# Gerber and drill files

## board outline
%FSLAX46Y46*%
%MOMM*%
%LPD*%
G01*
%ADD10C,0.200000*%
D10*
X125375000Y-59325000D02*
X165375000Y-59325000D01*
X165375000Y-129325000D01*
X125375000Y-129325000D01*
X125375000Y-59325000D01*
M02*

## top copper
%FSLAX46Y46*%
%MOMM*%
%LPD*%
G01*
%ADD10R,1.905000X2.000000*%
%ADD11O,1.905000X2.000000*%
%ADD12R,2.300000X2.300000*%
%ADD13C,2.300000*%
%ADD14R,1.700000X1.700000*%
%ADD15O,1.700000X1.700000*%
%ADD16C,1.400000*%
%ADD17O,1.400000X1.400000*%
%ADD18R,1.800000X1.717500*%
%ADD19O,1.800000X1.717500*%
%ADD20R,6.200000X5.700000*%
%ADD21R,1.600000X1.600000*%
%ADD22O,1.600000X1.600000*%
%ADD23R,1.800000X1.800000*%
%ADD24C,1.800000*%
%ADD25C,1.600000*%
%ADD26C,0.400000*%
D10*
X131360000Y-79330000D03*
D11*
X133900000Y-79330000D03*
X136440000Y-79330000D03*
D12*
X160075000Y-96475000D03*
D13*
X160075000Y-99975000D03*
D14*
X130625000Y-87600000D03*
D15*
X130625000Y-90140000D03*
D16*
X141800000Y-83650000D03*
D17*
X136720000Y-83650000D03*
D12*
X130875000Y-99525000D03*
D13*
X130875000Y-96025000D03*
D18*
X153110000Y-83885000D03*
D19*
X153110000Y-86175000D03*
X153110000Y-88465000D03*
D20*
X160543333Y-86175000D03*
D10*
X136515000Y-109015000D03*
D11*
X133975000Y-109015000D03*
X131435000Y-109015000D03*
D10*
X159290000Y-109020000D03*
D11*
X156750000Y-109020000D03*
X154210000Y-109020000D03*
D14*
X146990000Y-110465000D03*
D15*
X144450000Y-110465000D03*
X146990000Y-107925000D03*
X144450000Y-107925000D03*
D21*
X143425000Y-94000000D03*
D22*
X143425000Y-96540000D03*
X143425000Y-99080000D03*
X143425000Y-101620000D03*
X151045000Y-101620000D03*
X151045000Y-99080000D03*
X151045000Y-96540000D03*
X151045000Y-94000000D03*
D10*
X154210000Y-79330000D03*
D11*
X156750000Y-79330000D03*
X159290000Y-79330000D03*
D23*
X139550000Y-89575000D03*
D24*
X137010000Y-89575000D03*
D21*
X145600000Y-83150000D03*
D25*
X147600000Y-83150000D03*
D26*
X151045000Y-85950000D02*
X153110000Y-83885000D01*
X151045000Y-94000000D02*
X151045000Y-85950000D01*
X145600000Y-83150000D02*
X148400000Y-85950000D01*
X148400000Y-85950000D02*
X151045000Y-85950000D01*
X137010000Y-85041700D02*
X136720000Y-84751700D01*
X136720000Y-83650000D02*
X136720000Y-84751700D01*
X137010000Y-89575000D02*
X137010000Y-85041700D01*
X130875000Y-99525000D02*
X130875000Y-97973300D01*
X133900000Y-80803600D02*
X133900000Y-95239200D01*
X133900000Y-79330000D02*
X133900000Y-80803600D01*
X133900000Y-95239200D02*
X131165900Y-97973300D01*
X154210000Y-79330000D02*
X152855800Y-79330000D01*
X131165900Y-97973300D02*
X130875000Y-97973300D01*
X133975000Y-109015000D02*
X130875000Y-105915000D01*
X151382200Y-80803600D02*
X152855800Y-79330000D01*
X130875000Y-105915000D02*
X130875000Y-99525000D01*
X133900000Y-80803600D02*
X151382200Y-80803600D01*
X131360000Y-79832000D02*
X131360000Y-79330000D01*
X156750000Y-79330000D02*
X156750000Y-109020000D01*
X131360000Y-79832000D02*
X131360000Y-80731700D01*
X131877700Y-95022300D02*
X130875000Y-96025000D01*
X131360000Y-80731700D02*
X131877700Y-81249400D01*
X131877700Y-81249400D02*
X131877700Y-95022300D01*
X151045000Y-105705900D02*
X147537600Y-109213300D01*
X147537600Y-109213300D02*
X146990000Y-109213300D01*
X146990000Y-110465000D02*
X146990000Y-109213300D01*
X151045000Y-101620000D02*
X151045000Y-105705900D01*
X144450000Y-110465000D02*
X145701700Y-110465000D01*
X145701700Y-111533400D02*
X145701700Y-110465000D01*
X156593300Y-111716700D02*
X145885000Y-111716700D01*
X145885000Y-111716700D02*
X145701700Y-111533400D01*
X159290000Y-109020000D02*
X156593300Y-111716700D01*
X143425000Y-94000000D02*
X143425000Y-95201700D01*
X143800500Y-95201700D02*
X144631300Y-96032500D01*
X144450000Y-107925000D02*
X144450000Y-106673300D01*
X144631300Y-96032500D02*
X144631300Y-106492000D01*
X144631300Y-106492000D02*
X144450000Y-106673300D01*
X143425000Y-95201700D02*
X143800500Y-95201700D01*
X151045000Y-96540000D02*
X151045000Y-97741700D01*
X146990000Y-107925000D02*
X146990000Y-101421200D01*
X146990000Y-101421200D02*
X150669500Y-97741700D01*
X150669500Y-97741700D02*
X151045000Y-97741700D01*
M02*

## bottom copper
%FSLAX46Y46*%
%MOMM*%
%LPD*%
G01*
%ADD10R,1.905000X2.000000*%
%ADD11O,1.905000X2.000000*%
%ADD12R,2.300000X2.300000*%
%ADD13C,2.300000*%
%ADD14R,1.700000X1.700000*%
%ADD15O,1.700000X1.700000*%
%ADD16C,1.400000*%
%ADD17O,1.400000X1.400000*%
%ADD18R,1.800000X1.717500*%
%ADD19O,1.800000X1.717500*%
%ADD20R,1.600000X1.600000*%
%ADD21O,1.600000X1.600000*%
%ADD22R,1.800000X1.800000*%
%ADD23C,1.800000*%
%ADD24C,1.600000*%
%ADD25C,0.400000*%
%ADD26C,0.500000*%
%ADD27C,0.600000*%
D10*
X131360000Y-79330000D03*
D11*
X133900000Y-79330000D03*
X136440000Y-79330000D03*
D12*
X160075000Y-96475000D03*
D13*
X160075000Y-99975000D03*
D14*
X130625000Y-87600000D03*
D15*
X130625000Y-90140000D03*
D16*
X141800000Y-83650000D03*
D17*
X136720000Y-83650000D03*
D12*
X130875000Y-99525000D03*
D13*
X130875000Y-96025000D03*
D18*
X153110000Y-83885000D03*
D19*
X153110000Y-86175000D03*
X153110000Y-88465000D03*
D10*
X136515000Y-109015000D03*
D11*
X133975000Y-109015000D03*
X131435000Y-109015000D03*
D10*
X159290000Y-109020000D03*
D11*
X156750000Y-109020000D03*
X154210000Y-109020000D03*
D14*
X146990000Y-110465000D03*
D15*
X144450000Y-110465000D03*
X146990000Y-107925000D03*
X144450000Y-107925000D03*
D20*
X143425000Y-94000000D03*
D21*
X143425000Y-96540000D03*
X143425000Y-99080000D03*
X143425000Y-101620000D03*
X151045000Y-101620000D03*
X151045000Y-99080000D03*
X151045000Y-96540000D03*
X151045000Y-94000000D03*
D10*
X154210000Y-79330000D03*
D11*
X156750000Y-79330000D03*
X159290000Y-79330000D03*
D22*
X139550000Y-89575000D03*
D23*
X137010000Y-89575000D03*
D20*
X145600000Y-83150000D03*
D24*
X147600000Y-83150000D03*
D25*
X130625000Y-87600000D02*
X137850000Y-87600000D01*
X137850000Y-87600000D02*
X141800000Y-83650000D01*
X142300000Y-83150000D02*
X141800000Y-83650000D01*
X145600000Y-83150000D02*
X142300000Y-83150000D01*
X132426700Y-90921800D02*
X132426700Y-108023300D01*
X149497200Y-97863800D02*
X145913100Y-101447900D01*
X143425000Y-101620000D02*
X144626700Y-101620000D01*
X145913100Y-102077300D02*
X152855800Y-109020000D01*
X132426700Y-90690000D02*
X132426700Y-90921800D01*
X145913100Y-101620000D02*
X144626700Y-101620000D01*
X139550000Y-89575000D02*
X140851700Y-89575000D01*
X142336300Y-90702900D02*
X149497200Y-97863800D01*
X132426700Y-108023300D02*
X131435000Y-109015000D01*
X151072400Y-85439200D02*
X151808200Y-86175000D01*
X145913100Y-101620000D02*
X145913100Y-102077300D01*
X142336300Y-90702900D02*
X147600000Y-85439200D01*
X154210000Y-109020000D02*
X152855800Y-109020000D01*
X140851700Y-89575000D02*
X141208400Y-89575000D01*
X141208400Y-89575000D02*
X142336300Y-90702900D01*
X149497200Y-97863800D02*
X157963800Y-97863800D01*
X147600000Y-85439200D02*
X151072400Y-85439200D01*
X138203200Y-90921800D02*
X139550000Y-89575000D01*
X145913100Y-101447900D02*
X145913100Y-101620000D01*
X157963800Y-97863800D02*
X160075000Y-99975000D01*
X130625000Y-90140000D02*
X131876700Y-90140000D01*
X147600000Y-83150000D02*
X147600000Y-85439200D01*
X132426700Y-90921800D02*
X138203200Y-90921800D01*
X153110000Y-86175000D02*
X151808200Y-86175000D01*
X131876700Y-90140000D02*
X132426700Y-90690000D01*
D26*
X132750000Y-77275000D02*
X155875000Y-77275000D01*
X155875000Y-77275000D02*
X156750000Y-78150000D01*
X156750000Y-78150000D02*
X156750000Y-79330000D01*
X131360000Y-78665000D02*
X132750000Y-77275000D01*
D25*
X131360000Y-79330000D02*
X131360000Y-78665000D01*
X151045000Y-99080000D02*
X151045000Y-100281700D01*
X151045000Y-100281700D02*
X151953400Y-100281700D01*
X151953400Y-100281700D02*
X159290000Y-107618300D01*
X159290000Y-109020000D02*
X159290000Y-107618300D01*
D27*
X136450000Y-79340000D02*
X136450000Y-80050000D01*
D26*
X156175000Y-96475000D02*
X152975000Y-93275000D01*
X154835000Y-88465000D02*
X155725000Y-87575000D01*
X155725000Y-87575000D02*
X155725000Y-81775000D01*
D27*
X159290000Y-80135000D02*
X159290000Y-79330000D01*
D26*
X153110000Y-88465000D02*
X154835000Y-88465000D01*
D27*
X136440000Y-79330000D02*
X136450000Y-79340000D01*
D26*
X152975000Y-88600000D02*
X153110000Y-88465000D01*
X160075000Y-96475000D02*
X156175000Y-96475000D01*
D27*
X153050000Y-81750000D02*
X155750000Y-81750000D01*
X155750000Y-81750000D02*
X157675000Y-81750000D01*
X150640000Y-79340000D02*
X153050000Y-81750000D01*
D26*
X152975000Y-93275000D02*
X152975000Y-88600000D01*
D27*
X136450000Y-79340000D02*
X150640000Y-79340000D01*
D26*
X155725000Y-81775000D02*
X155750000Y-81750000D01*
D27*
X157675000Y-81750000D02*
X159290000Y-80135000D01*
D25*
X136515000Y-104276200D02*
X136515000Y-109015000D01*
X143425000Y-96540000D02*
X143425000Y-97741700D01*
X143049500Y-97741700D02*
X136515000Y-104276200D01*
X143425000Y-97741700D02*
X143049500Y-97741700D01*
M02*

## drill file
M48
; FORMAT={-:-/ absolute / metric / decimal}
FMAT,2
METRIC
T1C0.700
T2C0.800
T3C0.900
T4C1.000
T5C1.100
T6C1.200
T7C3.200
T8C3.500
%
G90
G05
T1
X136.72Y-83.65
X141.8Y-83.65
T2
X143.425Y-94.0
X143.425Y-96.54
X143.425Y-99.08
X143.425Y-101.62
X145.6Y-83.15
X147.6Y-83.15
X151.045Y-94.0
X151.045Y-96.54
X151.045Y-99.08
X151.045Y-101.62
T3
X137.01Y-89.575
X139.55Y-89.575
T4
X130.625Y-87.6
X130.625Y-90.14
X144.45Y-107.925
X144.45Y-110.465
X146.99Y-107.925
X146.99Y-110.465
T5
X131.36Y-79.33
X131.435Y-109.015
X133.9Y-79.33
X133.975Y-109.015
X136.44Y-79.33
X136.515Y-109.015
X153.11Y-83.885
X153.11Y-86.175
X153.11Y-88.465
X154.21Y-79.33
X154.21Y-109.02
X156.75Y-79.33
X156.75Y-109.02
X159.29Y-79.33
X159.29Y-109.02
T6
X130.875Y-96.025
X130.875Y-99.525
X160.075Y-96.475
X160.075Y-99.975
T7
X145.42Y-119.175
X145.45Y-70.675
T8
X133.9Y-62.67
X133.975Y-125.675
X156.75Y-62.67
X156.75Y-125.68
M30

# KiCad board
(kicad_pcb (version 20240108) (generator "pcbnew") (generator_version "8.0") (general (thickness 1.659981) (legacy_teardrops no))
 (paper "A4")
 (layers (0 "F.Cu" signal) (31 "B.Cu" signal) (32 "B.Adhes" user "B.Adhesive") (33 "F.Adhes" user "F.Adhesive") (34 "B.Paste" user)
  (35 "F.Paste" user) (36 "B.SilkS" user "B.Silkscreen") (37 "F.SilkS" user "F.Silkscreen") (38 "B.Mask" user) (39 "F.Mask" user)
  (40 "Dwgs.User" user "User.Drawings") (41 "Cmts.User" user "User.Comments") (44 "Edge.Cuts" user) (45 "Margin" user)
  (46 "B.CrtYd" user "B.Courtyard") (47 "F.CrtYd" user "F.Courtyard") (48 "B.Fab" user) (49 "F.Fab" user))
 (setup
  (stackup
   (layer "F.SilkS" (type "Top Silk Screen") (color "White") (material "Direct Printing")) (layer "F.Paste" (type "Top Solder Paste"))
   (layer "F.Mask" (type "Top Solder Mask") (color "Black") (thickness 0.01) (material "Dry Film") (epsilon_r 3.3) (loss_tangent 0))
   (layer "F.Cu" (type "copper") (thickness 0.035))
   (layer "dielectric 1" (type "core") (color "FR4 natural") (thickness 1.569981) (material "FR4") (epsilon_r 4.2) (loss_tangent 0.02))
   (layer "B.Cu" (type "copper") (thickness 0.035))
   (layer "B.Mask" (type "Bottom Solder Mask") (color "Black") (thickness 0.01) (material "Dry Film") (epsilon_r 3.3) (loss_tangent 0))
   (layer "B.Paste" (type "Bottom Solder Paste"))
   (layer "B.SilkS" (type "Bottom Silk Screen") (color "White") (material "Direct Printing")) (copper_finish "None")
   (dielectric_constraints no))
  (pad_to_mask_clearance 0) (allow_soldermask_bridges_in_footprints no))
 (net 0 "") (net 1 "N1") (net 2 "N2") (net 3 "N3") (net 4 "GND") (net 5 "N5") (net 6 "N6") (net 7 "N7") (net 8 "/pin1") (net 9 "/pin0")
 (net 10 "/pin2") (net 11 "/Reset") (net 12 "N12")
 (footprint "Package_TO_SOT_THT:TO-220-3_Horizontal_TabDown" (layer "F.Cu") (at 131.36 79.33)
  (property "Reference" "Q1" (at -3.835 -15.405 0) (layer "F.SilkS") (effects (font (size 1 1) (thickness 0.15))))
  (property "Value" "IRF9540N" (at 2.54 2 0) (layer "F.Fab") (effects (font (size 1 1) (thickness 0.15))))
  (pad "" np_thru_hole oval (at 2.54 -16.66) (size 3.5 3.5) (drill 3.5) (layers "*.Cu" "*.Mask"))
  (pad "1" thru_hole rect (at 0 0) (size 1.905 2) (drill 1.1) (layers "*.Cu" "*.Mask") (remove_unused_layers no) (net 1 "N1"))
  (pad "2" thru_hole oval (at 2.54 0) (size 1.905 2) (drill 1.1) (layers "*.Cu" "*.Mask") (remove_unused_layers no) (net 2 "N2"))
  (pad "3" thru_hole oval (at 5.08 0) (size 1.905 2) (drill 1.1) (layers "*.Cu" "*.Mask") (remove_unused_layers no) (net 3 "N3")))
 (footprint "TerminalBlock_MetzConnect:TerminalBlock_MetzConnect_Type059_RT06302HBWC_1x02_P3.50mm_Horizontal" (layer "F.Cu")
  (at 160.075 96.475 -90)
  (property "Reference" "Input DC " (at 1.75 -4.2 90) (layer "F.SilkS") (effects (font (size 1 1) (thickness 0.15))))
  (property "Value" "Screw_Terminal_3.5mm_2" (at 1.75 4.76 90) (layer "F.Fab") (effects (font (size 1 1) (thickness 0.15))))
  (pad "1" thru_hole rect (at 0 0 270) (size 2.3 2.3) (drill 1.2) (layers "*.Cu" "*.Mask") (remove_unused_layers no) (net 3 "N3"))
  (pad "2" thru_hole circle (at 3.5 0 270) (size 2.3 2.3) (drill 1.2) (layers "*.Cu" "*.Mask") (remove_unused_layers no) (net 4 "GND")))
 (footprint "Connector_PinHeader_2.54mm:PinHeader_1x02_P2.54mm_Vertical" (layer "F.Cu") (at 130.625 87.6)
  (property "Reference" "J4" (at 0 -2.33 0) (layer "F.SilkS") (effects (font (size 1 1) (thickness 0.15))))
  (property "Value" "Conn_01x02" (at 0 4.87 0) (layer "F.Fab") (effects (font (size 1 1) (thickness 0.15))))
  (pad "1" thru_hole rect (at 0 0) (size 1.7 1.7) (drill 1) (layers "*.Cu" "*.Mask") (remove_unused_layers no) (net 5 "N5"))
  (pad "2" thru_hole oval (at 0 2.54) (size 1.7 1.7) (drill 1) (layers "*.Cu" "*.Mask") (remove_unused_layers no) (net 4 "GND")))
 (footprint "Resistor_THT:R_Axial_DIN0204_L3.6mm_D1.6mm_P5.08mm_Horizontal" (layer "F.Cu") (at 141.8 83.65 180)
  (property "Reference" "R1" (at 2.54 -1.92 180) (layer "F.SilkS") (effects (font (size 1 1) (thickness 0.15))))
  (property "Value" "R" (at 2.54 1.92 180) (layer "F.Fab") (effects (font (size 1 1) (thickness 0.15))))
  (pad "1" thru_hole circle (at 0 0 180) (size 1.4 1.4) (drill 0.7) (layers "*.Cu" "*.Mask") (remove_unused_layers no) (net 5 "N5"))
  (pad "2" thru_hole oval (at 5.08 0 180) (size 1.4 1.4) (drill 0.7) (layers "*.Cu" "*.Mask") (remove_unused_layers no) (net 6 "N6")))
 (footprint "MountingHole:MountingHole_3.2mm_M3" (layer "F.Cu") (at 145.42 119.175)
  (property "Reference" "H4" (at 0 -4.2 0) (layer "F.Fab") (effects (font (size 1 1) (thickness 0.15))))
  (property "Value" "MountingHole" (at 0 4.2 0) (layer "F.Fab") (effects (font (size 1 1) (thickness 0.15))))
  (pad "" np_thru_hole circle (at 0 0) (size 3.2 3.2) (drill 3.2) (layers "*.Cu" "*.Mask")))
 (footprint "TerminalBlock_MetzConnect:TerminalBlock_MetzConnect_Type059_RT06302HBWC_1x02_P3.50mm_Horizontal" (layer "F.Cu")
  (at 130.875 99.525 90)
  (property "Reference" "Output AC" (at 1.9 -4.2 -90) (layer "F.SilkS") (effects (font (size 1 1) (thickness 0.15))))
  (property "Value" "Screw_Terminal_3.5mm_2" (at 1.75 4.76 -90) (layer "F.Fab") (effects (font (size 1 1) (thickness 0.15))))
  (pad "1" thru_hole rect (at 0 0 90) (size 2.3 2.3) (drill 1.2) (layers "*.Cu" "*.Mask") (remove_unused_layers no) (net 2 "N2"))
  (pad "2" thru_hole circle (at 3.5 0 90) (size 2.3 2.3) (drill 1.2) (layers "*.Cu" "*.Mask") (remove_unused_layers no) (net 1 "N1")))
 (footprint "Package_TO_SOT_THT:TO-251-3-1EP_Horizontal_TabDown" (layer "F.Cu") (at 153.11 83.885 -90)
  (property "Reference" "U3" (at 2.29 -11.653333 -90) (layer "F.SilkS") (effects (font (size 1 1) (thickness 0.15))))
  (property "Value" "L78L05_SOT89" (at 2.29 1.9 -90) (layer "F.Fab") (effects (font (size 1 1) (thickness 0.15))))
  (pad "1" thru_hole rect (at 0 0 270) (size 1.7175 1.8) (drill 1.1) (layers "*.Cu" "*.Mask") (remove_unused_layers no) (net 5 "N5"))
  (pad "2" thru_hole oval (at 2.29 0 270) (size 1.7175 1.8) (drill 1.1) (layers "*.Cu" "*.Mask") (remove_unused_layers no) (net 4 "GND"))
  (pad "3" thru_hole oval (at 4.58 0 270) (size 1.7175 1.8) (drill 1.1) (layers "*.Cu" "*.Mask") (remove_unused_layers no) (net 3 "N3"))
  (pad "4" smd rect (at 2.29 -7.433333 270) (size 5.7 6.2) (layers "F.Cu" "F.Paste" "F.Mask")))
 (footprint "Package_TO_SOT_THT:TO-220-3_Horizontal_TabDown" (layer "F.Cu") (at 136.515 109.015 180)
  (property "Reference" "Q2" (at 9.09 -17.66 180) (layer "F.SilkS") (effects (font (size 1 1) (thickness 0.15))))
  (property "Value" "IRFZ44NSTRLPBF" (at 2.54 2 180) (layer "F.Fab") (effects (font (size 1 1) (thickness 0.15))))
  (pad "" np_thru_hole oval (at 2.54 -16.66 180) (size 3.5 3.5) (drill 3.5) (layers "*.Cu" "*.Mask"))
  (pad "1" thru_hole rect (at 0 0 180) (size 1.905 2) (drill 1.1) (layers "*.Cu" "*.Mask") (remove_unused_layers no) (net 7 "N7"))
  (pad "2" thru_hole oval (at 2.54 0 180) (size 1.905 2) (drill 1.1) (layers "*.Cu" "*.Mask") (remove_unused_layers no) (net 2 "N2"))
  (pad "3" thru_hole oval (at 5.08 0 180) (size 1.905 2) (drill 1.1) (layers "*.Cu" "*.Mask") (remove_unused_layers no) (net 4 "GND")))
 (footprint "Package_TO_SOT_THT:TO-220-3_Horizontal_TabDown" (layer "F.Cu") (at 159.29 109.02 180)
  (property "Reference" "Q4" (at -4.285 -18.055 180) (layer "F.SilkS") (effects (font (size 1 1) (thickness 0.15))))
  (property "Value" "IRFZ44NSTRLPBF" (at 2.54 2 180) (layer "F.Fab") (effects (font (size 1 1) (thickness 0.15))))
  (pad "" np_thru_hole oval (at 2.54 -16.66 180) (size 3.5 3.5) (drill 3.5) (layers "*.Cu" "*.Mask"))
  (pad "1" thru_hole rect (at 0 0 180) (size 1.905 2) (drill 1.1) (layers "*.Cu" "*.Mask") (remove_unused_layers no) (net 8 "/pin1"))
  (pad "2" thru_hole oval (at 2.54 0 180) (size 1.905 2) (drill 1.1) (layers "*.Cu" "*.Mask") (remove_unused_layers no) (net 1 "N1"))
  (pad "3" thru_hole oval (at 5.08 0 180) (size 1.905 2) (drill 1.1) (layers "*.Cu" "*.Mask") (remove_unused_layers no) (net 4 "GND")))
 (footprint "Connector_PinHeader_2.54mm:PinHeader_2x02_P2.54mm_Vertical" (layer "F.Cu") (at 146.99 110.465 180)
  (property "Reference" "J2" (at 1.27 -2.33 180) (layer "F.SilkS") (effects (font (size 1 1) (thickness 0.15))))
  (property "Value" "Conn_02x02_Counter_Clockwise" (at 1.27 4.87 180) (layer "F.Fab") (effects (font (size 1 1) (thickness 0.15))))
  (pad "1" thru_hole rect (at 0 0 180) (size 1.7 1.7) (drill 1) (layers "*.Cu" "*.Mask") (remove_unused_layers no) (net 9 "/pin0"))
  (pad "2" thru_hole oval (at 2.54 0 180) (size 1.7 1.7) (drill 1) (layers "*.Cu" "*.Mask") (remove_unused_layers no) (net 8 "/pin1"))
  (pad "3" thru_hole oval (at 0 2.54 180) (size 1.7 1.7) (drill 1) (layers "*.Cu" "*.Mask") (remove_unused_layers no) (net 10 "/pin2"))
  (pad "4" thru_hole oval (at 2.54 2.54 180) (size 1.7 1.7) (drill 1) (layers "*.Cu" "*.Mask") (remove_unused_layers no) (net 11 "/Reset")))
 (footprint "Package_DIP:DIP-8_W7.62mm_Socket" (layer "F.Cu") (at 143.425 94)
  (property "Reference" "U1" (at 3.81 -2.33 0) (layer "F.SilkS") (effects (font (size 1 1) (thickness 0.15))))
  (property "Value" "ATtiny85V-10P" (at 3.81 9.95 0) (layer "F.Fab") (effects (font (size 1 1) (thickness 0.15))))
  (pad "1" thru_hole rect (at 0 0) (size 1.6 1.6) (drill 0.8) (layers "*.Cu" "*.Mask") (remove_unused_layers no) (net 11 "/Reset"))
  (pad "2" thru_hole oval (at 0 2.54) (size 1.6 1.6) (drill 0.8) (layers "*.Cu" "*.Mask") (remove_unused_layers no) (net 7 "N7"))
  (pad "3" thru_hole oval (at 0 5.08) (size 1.6 1.6) (drill 0.8) (layers "*.Cu" "*.Mask") (remove_unused_layers no) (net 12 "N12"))
  (pad "4" thru_hole oval (at 0 7.62) (size 1.6 1.6) (drill 0.8) (layers "*.Cu" "*.Mask") (remove_unused_layers no) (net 4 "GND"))
  (pad "5" thru_hole oval (at 7.62 7.62) (size 1.6 1.6) (drill 0.8) (layers "*.Cu" "*.Mask") (remove_unused_layers no) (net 9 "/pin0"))
  (pad "6" thru_hole oval (at 7.62 5.08) (size 1.6 1.6) (drill 0.8) (layers "*.Cu" "*.Mask") (remove_unused_layers no) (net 8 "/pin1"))
  (pad "7" thru_hole oval (at 7.62 2.54) (size 1.6 1.6) (drill 0.8) (layers "*.Cu" "*.Mask") (remove_unused_layers no) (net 10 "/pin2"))
  (pad "8" thru_hole oval (at 7.62 0) (size 1.6 1.6) (drill 0.8) (layers "*.Cu" "*.Mask") (remove_unused_layers no) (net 5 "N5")))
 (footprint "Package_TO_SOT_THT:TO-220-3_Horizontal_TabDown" (layer "F.Cu") (at 154.21 79.33)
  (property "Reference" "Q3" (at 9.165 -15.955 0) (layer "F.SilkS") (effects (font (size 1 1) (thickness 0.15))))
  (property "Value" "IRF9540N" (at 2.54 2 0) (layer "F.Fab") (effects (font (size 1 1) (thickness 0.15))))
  (pad "" np_thru_hole oval (at 2.54 -16.66) (size 3.5 3.5) (drill 3.5) (layers "*.Cu" "*.Mask"))
  (pad "1" thru_hole rect (at 0 0) (size 1.905 2) (drill 1.1) (layers "*.Cu" "*.Mask") (remove_unused_layers no) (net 2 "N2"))
  (pad "2" thru_hole oval (at 2.54 0) (size 1.905 2) (drill 1.1) (layers "*.Cu" "*.Mask") (remove_unused_layers no) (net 1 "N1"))
  (pad "3" thru_hole oval (at 5.08 0) (size 1.905 2) (drill 1.1) (layers "*.Cu" "*.Mask") (remove_unused_layers no) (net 3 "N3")))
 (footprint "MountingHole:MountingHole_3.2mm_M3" (layer "F.Cu") (at 145.45 70.675)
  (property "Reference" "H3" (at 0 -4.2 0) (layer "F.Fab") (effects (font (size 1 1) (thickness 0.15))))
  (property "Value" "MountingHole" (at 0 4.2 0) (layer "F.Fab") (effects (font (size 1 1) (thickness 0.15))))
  (pad "" np_thru_hole circle (at 0 0) (size 3.2 3.2) (drill 3.2) (layers "*.Cu" "*.Mask")))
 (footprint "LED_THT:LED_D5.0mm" (layer "F.Cu") (at 139.55 89.575 180)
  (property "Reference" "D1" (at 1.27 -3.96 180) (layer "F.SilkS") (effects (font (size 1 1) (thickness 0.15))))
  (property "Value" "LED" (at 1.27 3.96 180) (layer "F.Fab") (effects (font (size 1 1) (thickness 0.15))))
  (pad "1" thru_hole rect (at 0 0 180) (size 1.8 1.8) (drill 0.9) (layers "*.Cu" "*.Mask") (remove_unused_layers no) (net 4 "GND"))
  (pad "2" thru_hole circle (at 2.54 0 180) (size 1.8 1.8) (drill 0.9) (layers "*.Cu" "*.Mask") (remove_unused_layers no) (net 6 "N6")))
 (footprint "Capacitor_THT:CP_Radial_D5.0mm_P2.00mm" (layer "F.Cu") (at 145.6 83.15)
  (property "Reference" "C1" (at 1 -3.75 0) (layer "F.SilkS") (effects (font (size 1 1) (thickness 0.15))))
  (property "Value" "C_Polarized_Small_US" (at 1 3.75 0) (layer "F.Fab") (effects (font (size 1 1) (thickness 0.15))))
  (pad "1" thru_hole rect (at 0 0) (size 1.6 1.6) (drill 0.8) (layers "*.Cu" "*.Mask") (remove_unused_layers no) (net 5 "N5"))
  (pad "2" thru_hole circle (at 2 0) (size 1.6 1.6) (drill 0.8) (layers "*.Cu" "*.Mask") (remove_unused_layers no) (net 4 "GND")))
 (gr_rect (start 125.375 59.325) (end 165.375 129.325) (stroke (width 0.2) (type default)) (fill none) (layer "Edge.Cuts"))
 (segment (start 151.045 85.95) (end 153.11 83.885) (width 0.4) (layer "F.Cu") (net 5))
 (segment (start 151.045 94) (end 151.045 85.95) (width 0.4) (layer "F.Cu") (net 5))
 (segment (start 145.6 83.15) (end 148.4 85.95) (width 0.4) (layer "F.Cu") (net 5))
 (segment (start 148.4 85.95) (end 151.045 85.95) (width 0.4) (layer "F.Cu") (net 5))
 (segment (start 130.625 87.6) (end 137.85 87.6) (width 0.4) (layer "B.Cu") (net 5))
 (segment (start 137.85 87.6) (end 141.8 83.65) (width 0.4) (layer "B.Cu") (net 5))
 (segment (start 142.3 83.15) (end 141.8 83.65) (width 0.4) (layer "B.Cu") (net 5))
 (segment (start 145.6 83.15) (end 142.3 83.15) (width 0.4) (layer "B.Cu") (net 5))
 (segment (start 132.4267 90.9218) (end 132.4267 108.0233) (width 0.4) (layer "B.Cu") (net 4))
 (segment (start 149.4972 97.8638) (end 145.9131 101.4479) (width 0.4) (layer "B.Cu") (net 4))
 (segment (start 143.425 101.62) (end 144.6267 101.62) (width 0.4) (layer "B.Cu") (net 4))
 (segment (start 145.9131 102.0773) (end 152.8558 109.02) (width 0.4) (layer "B.Cu") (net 4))
 (segment (start 132.4267 90.69) (end 132.4267 90.9218) (width 0.4) (layer "B.Cu") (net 4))
 (segment (start 145.9131 101.62) (end 144.6267 101.62) (width 0.4) (layer "B.Cu") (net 4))
 (segment (start 139.55 89.575) (end 140.8517 89.575) (width 0.4) (layer "B.Cu") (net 4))
 (segment (start 142.3363 90.7029) (end 149.4972 97.8638) (width 0.4) (layer "B.Cu") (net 4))
 (segment (start 132.4267 108.0233) (end 131.435 109.015) (width 0.4) (layer "B.Cu") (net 4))
 (segment (start 151.0724 85.4392) (end 151.8082 86.175) (width 0.4) (layer "B.Cu") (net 4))
 (segment (start 145.9131 101.62) (end 145.9131 102.0773) (width 0.4) (layer "B.Cu") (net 4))
 (segment (start 142.3363 90.7029) (end 147.6 85.4392) (width 0.4) (layer "B.Cu") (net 4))
 (segment (start 154.21 109.02) (end 152.8558 109.02) (width 0.4) (layer "B.Cu") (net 4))
 (segment (start 140.8517 89.575) (end 141.2084 89.575) (width 0.4) (layer "B.Cu") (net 4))
 (segment (start 141.2084 89.575) (end 142.3363 90.7029) (width 0.4) (layer "B.Cu") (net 4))
 (segment (start 149.4972 97.8638) (end 157.9638 97.8638) (width 0.4) (layer "B.Cu") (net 4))
 (segment (start 147.6 85.4392) (end 151.0724 85.4392) (width 0.4) (layer "B.Cu") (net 4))
 (segment (start 138.2032 90.9218) (end 139.55 89.575) (width 0.4) (layer "B.Cu") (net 4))
 (segment (start 145.9131 101.4479) (end 145.9131 101.62) (width 0.4) (layer "B.Cu") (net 4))
 (segment (start 157.9638 97.8638) (end 160.075 99.975) (width 0.4) (layer "B.Cu") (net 4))
 (segment (start 130.625 90.14) (end 131.8767 90.14) (width 0.4) (layer "B.Cu") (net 4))
 (segment (start 147.6 83.15) (end 147.6 85.4392) (width 0.4) (layer "B.Cu") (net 4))
 (segment (start 132.4267 90.9218) (end 138.2032 90.9218) (width 0.4) (layer "B.Cu") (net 4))
 (segment (start 153.11 86.175) (end 151.8082 86.175) (width 0.4) (layer "B.Cu") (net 4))
 (segment (start 131.8767 90.14) (end 132.4267 90.69) (width 0.4) (layer "B.Cu") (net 4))
 (segment (start 137.01 85.0417) (end 136.72 84.7517) (width 0.4) (layer "F.Cu") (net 6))
 (segment (start 136.72 83.65) (end 136.72 84.7517) (width 0.4) (layer "F.Cu") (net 6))
 (segment (start 137.01 89.575) (end 137.01 85.0417) (width 0.4) (layer "F.Cu") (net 6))
 (segment (start 130.875 99.525) (end 130.875 97.9733) (width 0.4) (layer "F.Cu") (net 2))
 (segment (start 133.9 80.8036) (end 133.9 95.2392) (width 0.4) (layer "F.Cu") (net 2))
 (segment (start 133.9 79.33) (end 133.9 80.8036) (width 0.4) (layer "F.Cu") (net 2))
 (segment (start 133.9 95.2392) (end 131.1659 97.9733) (width 0.4) (layer "F.Cu") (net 2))
 (segment (start 154.21 79.33) (end 152.8558 79.33) (width 0.4) (layer "F.Cu") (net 2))
 (segment (start 131.1659 97.9733) (end 130.875 97.9733) (width 0.4) (layer "F.Cu") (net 2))
 (segment (start 133.975 109.015) (end 130.875 105.915) (width 0.4) (layer "F.Cu") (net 2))
 (segment (start 151.3822 80.8036) (end 152.8558 79.33) (width 0.4) (layer "F.Cu") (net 2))
 (segment (start 130.875 105.915) (end 130.875 99.525) (width 0.4) (layer "F.Cu") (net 2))
 (segment (start 133.9 80.8036) (end 151.3822 80.8036) (width 0.4) (layer "F.Cu") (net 2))
 (segment (start 131.36 79.832) (end 131.36 79.33) (width 0.4) (layer "F.Cu") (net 1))
 (segment (start 156.75 79.33) (end 156.75 109.02) (width 0.4) (layer "F.Cu") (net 1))
 (segment (start 131.36 79.832) (end 131.36 80.7317) (width 0.4) (layer "F.Cu") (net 1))
 (segment (start 131.8777 95.0223) (end 130.875 96.025) (width 0.4) (layer "F.Cu") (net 1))
 (segment (start 131.36 80.7317) (end 131.8777 81.2494) (width 0.4) (layer "F.Cu") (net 1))
 (segment (start 131.8777 81.2494) (end 131.8777 95.0223) (width 0.4) (layer "F.Cu") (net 1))
 (segment (start 132.75 77.275) (end 155.875 77.275) (width 0.5) (layer "B.Cu") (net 1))
 (segment (start 155.875 77.275) (end 156.75 78.15) (width 0.5) (layer "B.Cu") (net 1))
 (segment (start 156.75 78.15) (end 156.75 79.33) (width 0.5) (layer "B.Cu") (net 1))
 (segment (start 131.36 78.665) (end 132.75 77.275) (width 0.5) (layer "B.Cu") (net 1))
 (segment (start 131.36 79.33) (end 131.36 78.665) (width 0.4) (layer "B.Cu") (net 1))
 (segment (start 151.045 105.7059) (end 147.5376 109.2133) (width 0.4) (layer "F.Cu") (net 9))
 (segment (start 147.5376 109.2133) (end 146.99 109.2133) (width 0.4) (layer "F.Cu") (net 9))
 (segment (start 146.99 110.465) (end 146.99 109.2133) (width 0.4) (layer "F.Cu") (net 9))
 (segment (start 151.045 101.62) (end 151.045 105.7059) (width 0.4) (layer "F.Cu") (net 9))
 (segment (start 144.45 110.465) (end 145.7017 110.465) (width 0.4) (layer "F.Cu") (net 8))
 (segment (start 145.7017 111.5334) (end 145.7017 110.465) (width 0.4) (layer "F.Cu") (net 8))
 (segment (start 156.5933 111.7167) (end 145.885 111.7167) (width 0.4) (layer "F.Cu") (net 8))
 (segment (start 145.885 111.7167) (end 145.7017 111.5334) (width 0.4) (layer "F.Cu") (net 8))
 (segment (start 159.29 109.02) (end 156.5933 111.7167) (width 0.4) (layer "F.Cu") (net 8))
 (segment (start 151.045 99.08) (end 151.045 100.2817) (width 0.4) (layer "B.Cu") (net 8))
 (segment (start 151.045 100.2817) (end 151.9534 100.2817) (width 0.4) (layer "B.Cu") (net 8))
 (segment (start 151.9534 100.2817) (end 159.29 107.6183) (width 0.4) (layer "B.Cu") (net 8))
 (segment (start 159.29 109.02) (end 159.29 107.6183) (width 0.4) (layer "B.Cu") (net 8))
 (segment (start 143.425 94) (end 143.425 95.2017) (width 0.4) (layer "F.Cu") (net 11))
 (segment (start 143.8005 95.2017) (end 144.6313 96.0325) (width 0.4) (layer "F.Cu") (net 11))
 (segment (start 144.45 107.925) (end 144.45 106.6733) (width 0.4) (layer "F.Cu") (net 11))
 (segment (start 144.6313 96.0325) (end 144.6313 106.492) (width 0.4) (layer "F.Cu") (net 11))
 (segment (start 144.6313 106.492) (end 144.45 106.6733) (width 0.4) (layer "F.Cu") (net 11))
 (segment (start 143.425 95.2017) (end 143.8005 95.2017) (width 0.4) (layer "F.Cu") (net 11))
 (segment (start 151.045 96.54) (end 151.045 97.7417) (width 0.4) (layer "F.Cu") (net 10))
 (segment (start 146.99 107.925) (end 146.99 101.4212) (width 0.4) (layer "F.Cu") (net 10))
 (segment (start 146.99 101.4212) (end 150.6695 97.7417) (width 0.4) (layer "F.Cu") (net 10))
 (segment (start 150.6695 97.7417) (end 151.045 97.7417) (width 0.4) (layer "F.Cu") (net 10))
 (segment (start 136.45 79.34) (end 136.45 80.05) (width 0.6) (layer "B.Cu") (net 3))
 (segment (start 156.175 96.475) (end 152.975 93.275) (width 0.5) (layer "B.Cu") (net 3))
 (segment (start 154.835 88.465) (end 155.725 87.575) (width 0.5) (layer "B.Cu") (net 3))
 (segment (start 155.725 87.575) (end 155.725 81.775) (width 0.5) (layer "B.Cu") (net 3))
 (segment (start 159.29 80.135) (end 159.29 79.33) (width 0.6) (layer "B.Cu") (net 3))
 (segment (start 153.11 88.465) (end 154.835 88.465) (width 0.5) (layer "B.Cu") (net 3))
 (segment (start 136.44 79.33) (end 136.45 79.34) (width 0.6) (layer "B.Cu") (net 3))
 (segment (start 152.975 88.6) (end 153.11 88.465) (width 0.5) (layer "B.Cu") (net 3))
 (segment (start 160.075 96.475) (end 156.175 96.475) (width 0.5) (layer "B.Cu") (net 3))
 (segment (start 153.05 81.75) (end 155.75 81.75) (width 0.6) (layer "B.Cu") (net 3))
 (segment (start 155.75 81.75) (end 157.675 81.75) (width 0.6) (layer "B.Cu") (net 3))
 (segment (start 150.64 79.34) (end 153.05 81.75) (width 0.6) (layer "B.Cu") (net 3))
 (segment (start 152.975 93.275) (end 152.975 88.6) (width 0.5) (layer "B.Cu") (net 3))
 (segment (start 136.45 79.34) (end 150.64 79.34) (width 0.6) (layer "B.Cu") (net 3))
 (segment (start 155.725 81.775) (end 155.75 81.75) (width 0.5) (layer "B.Cu") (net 3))
 (segment (start 157.675 81.75) (end 159.29 80.135) (width 0.6) (layer "B.Cu") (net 3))
 (segment (start 136.515 104.2762) (end 136.515 109.015) (width 0.4) (layer "B.Cu") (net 7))
 (segment (start 143.425 96.54) (end 143.425 97.7417) (width 0.4) (layer "B.Cu") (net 7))
 (segment (start 143.0495 97.7417) (end 136.515 104.2762) (width 0.4) (layer "B.Cu") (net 7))
 (segment (start 143.425 97.7417) (end 143.0495 97.7417) (width 0.4) (layer "B.Cu") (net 7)))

